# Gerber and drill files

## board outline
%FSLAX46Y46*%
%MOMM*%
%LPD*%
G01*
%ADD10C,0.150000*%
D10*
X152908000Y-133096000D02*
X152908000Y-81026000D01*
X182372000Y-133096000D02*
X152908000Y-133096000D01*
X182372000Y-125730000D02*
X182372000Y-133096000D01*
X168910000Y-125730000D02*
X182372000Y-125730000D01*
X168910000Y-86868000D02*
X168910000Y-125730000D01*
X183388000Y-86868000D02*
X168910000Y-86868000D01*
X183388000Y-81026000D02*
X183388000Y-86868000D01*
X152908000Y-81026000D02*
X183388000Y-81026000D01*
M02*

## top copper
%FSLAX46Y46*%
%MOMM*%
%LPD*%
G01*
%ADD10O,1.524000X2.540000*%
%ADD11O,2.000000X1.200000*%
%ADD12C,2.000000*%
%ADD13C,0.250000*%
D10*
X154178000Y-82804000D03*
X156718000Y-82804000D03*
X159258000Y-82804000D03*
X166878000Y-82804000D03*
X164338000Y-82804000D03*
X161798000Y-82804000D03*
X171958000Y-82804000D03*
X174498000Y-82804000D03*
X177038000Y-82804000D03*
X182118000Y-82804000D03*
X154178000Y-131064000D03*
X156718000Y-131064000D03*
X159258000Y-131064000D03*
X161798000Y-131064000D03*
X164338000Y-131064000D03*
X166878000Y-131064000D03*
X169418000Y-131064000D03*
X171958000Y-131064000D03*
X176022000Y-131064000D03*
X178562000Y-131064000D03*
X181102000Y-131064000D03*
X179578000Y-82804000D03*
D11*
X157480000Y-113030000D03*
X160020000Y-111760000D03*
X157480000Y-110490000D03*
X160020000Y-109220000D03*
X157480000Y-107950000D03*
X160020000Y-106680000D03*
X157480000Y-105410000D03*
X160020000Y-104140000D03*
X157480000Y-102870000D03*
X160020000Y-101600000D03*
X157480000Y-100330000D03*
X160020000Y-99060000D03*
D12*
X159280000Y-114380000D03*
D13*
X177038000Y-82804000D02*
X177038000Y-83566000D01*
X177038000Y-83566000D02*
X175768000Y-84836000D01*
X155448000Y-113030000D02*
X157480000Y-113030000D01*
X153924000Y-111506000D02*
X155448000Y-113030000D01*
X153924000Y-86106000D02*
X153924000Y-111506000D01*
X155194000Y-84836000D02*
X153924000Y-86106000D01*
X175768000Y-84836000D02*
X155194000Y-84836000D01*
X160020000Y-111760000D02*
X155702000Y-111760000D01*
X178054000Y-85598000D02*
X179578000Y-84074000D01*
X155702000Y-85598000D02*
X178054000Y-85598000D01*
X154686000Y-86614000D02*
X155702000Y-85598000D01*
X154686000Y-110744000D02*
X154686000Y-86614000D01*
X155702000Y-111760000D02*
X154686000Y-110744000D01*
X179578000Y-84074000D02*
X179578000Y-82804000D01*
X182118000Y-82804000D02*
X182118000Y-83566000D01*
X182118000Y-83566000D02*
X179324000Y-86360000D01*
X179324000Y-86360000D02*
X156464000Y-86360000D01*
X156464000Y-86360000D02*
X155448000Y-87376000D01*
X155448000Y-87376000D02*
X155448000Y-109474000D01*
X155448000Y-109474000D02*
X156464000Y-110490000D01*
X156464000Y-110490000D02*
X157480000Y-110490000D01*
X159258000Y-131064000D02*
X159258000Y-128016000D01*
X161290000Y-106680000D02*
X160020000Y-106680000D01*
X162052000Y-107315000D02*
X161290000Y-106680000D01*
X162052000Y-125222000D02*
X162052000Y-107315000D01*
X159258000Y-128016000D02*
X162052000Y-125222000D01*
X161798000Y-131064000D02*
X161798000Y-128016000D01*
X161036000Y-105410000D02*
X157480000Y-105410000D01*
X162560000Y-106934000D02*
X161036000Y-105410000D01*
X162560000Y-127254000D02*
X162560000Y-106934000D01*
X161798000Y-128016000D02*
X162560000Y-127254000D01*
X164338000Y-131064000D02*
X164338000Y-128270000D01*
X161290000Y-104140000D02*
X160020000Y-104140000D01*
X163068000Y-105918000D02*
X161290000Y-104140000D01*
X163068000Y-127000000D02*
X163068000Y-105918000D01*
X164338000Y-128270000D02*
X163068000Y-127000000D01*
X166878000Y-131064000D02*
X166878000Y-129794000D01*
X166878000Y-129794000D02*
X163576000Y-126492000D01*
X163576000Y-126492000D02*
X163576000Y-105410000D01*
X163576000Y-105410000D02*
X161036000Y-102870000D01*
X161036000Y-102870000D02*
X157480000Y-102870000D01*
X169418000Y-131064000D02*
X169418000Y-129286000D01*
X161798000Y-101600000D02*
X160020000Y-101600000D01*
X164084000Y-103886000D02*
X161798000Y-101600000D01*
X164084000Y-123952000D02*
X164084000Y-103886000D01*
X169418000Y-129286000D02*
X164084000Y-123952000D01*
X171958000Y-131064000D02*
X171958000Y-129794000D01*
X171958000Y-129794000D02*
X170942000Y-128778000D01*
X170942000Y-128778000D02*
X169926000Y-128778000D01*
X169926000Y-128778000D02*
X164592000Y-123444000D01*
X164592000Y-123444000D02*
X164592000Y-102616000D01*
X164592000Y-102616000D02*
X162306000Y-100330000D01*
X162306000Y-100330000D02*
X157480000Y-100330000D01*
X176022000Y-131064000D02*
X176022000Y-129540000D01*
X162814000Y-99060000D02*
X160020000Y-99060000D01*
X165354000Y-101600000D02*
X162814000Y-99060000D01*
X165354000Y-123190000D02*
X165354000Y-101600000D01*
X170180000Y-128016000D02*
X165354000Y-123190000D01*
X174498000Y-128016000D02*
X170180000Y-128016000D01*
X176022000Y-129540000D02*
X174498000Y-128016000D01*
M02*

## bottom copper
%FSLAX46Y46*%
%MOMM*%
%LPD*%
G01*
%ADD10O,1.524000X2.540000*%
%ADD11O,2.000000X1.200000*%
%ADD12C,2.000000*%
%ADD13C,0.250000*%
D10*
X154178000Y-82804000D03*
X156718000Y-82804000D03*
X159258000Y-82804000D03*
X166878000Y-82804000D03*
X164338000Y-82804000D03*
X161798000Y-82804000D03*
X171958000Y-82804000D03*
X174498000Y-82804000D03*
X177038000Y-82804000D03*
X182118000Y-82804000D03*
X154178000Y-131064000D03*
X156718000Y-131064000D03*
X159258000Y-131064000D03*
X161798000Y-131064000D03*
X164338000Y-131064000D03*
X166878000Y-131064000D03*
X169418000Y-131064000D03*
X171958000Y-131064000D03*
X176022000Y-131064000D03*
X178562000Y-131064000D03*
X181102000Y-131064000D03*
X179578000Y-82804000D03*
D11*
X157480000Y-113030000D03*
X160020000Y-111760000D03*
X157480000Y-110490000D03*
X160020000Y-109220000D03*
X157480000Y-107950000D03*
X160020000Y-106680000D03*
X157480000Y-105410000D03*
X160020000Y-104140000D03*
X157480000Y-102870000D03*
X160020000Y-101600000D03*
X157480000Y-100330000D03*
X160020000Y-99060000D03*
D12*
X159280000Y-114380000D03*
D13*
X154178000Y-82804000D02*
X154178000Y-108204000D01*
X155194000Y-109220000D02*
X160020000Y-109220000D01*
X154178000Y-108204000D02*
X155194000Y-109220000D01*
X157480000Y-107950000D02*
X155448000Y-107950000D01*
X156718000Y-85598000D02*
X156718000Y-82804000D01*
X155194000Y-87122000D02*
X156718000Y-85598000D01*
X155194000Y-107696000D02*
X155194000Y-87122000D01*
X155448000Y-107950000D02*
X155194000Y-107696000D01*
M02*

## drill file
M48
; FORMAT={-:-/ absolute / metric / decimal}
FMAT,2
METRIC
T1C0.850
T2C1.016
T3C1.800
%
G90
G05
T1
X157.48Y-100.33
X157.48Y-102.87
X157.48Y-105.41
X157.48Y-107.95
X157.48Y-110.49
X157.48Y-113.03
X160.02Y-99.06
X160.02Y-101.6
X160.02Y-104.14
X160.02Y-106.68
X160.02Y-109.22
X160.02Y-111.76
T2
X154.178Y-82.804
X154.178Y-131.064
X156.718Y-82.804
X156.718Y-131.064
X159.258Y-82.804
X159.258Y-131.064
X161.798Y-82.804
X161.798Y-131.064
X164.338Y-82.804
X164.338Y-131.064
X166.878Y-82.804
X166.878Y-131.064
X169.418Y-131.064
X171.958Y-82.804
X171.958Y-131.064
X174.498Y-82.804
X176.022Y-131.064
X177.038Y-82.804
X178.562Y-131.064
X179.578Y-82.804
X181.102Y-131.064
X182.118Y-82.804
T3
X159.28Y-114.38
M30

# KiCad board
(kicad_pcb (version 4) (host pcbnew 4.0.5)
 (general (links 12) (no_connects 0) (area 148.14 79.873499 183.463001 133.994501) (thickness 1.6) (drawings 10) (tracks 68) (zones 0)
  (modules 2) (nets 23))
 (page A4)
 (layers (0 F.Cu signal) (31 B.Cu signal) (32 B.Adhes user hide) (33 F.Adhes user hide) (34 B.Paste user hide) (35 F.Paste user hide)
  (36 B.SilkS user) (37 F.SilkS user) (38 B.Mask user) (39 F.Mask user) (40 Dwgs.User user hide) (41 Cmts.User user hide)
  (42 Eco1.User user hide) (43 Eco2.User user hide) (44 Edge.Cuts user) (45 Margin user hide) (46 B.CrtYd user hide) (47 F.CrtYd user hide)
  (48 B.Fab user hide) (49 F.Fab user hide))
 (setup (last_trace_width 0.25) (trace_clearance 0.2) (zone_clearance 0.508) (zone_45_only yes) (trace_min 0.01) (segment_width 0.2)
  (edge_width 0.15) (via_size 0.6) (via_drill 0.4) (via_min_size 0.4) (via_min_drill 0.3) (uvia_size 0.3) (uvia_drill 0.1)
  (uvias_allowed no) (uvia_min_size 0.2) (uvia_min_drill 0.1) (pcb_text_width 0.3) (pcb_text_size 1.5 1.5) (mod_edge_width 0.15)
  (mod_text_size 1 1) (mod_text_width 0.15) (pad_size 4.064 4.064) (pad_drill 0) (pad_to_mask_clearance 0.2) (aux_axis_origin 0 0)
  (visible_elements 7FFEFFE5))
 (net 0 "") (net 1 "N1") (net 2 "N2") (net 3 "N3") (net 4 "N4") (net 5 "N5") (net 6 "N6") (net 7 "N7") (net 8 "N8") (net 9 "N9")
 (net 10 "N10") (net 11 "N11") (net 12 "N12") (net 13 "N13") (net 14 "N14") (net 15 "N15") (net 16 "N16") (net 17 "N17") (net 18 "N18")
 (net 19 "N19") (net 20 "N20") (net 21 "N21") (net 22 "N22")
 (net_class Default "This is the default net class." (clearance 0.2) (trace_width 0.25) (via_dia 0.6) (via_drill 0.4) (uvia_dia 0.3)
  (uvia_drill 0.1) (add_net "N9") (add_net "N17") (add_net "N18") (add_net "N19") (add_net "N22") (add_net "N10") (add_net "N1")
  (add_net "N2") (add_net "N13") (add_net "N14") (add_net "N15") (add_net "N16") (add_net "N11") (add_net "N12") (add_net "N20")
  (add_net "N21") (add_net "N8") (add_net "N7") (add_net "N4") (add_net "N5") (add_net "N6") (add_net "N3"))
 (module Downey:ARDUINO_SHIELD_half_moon (layer F.Cu) (at 148.59 104.14 270)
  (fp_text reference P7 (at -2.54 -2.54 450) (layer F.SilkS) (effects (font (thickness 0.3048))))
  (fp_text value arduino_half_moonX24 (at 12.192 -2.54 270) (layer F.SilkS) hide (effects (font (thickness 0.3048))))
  (pad 11 thru_hole oval (at -21.336 -5.588 270) (size 2.54 1.524) (drill 1.016) (layers *.Cu *.Mask F.SilkS) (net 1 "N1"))
  (pad 10 thru_hole oval (at -21.336 -8.128 270) (size 2.54 1.524) (drill 1.016) (layers *.Cu *.Mask F.SilkS) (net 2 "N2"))
  (pad 9 thru_hole oval (at -21.336 -10.668 270) (size 2.54 1.524) (drill 1.016) (layers *.Cu *.Mask F.SilkS) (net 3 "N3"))
  (pad 6 thru_hole oval (at -21.336 -18.288 270) (size 2.54 1.524) (drill 1.016) (layers *.Cu *.Mask F.SilkS) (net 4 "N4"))
  (pad 7 thru_hole oval (at -21.336 -15.748 270) (size 2.54 1.524) (drill 1.016) (layers *.Cu *.Mask F.SilkS) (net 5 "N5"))
  (pad 8 thru_hole oval (at -21.336 -13.208 270) (size 2.54 1.524) (drill 1.016) (layers *.Cu *.Mask F.SilkS) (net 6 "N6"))
  (pad 5 thru_hole oval (at -21.336 -23.368 270) (size 2.54 1.524) (drill 1.016) (layers *.Cu *.Mask F.SilkS) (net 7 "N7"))
  (pad 4 thru_hole oval (at -21.336 -25.908 270) (size 2.54 1.524) (drill 1.016) (layers *.Cu *.Mask F.SilkS) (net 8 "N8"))
  (pad 3 thru_hole oval (at -21.336 -28.448 270) (size 2.54 1.524) (drill 1.016) (layers *.Cu *.Mask F.SilkS) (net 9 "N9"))
  (pad 1 thru_hole oval (at -21.336 -33.528 270) (size 2.54 1.524) (drill 1.016) (layers *.Cu *.Mask F.SilkS) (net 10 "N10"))
  (pad 12 thru_hole oval (at 26.924 -5.588 270) (size 2.54 1.524) (drill 1.016) (layers *.Cu *.Mask F.SilkS) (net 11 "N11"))
  (pad 13 thru_hole oval (at 26.924 -8.128 270) (size 2.54 1.524) (drill 1.016) (layers *.Cu *.Mask F.SilkS) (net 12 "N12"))
  (pad 14 thru_hole oval (at 26.924 -10.668 270) (size 2.54 1.524) (drill 1.016) (layers *.Cu *.Mask F.SilkS) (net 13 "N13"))
  (pad 15 thru_hole oval (at 26.924 -13.208 270) (size 2.54 1.524) (drill 1.016) (layers *.Cu *.Mask F.SilkS) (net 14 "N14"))
  (pad 16 thru_hole oval (at 26.924 -15.748 270) (size 2.54 1.524) (drill 1.016) (layers *.Cu *.Mask F.SilkS) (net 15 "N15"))
  (pad 17 thru_hole oval (at 26.924 -18.288 270) (size 2.54 1.524) (drill 1.016) (layers *.Cu *.Mask F.SilkS) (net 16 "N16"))
  (pad 18 thru_hole oval (at 26.924 -20.828 270) (size 2.54 1.524) (drill 1.016) (layers *.Cu *.Mask F.SilkS) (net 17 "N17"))
  (pad 19 thru_hole oval (at 26.924 -23.368 270) (size 2.54 1.524) (drill 1.016) (layers *.Cu *.Mask F.SilkS) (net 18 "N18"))
  (pad 20 thru_hole oval (at 26.924 -27.432 270) (size 2.54 1.524) (drill 1.016) (layers *.Cu *.Mask F.SilkS) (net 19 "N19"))
  (pad 21 thru_hole oval (at 26.924 -29.972 270) (size 2.54 1.524) (drill 1.016) (layers *.Cu *.Mask F.SilkS) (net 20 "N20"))
  (pad 22 thru_hole oval (at 26.924 -32.512 270) (size 2.54 1.524) (drill 1.016) (layers *.Cu *.Mask F.SilkS) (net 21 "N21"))
  (pad 2 thru_hole oval (at -21.336 -30.988 270) (size 2.54 1.524) (drill 1.016) (layers *.Cu *.Mask F.SilkS) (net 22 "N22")))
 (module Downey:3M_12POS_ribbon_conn (layer F.Cu) (at 158.75 106.68 90)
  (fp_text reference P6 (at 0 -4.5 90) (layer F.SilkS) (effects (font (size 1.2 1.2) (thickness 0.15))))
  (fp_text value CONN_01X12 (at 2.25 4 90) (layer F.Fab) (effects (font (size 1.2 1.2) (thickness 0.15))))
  (pad 1 thru_hole oval (at -6.35 -1.27 90) (size 1.2 2) (drill 0.85) (layers *.Cu *.Mask) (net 9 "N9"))
  (pad 2 thru_hole oval (at -5.08 1.27 90) (size 1.2 2) (drill 0.85) (layers *.Cu *.Mask) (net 22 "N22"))
  (pad 3 thru_hole oval (at -3.81 -1.27 90) (size 1.2 2) (drill 0.85) (layers *.Cu *.Mask) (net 10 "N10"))
  (pad 4 thru_hole oval (at -2.54 1.27 90) (size 1.2 2) (drill 0.85) (layers *.Cu *.Mask) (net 1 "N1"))
  (pad 5 thru_hole oval (at -1.27 -1.27 90) (size 1.2 2) (drill 0.85) (layers *.Cu *.Mask) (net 2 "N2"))
  (pad 6 thru_hole oval (at 0 1.27 90) (size 1.2 2) (drill 0.85) (layers *.Cu *.Mask) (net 13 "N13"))
  (pad 7 thru_hole oval (at 1.27 -1.27 90) (size 1.2 2) (drill 0.85) (layers *.Cu *.Mask) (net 14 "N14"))
  (pad 8 thru_hole oval (at 2.54 1.27 90) (size 1.2 2) (drill 0.85) (layers *.Cu *.Mask) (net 15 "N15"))
  (pad 9 thru_hole oval (at 3.81 -1.27 90) (size 1.2 2) (drill 0.85) (layers *.Cu *.Mask) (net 16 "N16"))
  (pad 10 thru_hole oval (at 5.08 1.27 90) (size 1.2 2) (drill 0.85) (layers *.Cu *.Mask) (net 17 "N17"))
  (pad 11 thru_hole oval (at 6.35 -1.27 90) (size 1.2 2) (drill 0.85) (layers *.Cu *.Mask) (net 18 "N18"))
  (pad 12 thru_hole oval (at 7.62 1.27 90) (size 1.2 2) (drill 0.85) (layers *.Cu *.Mask) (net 19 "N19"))
  (pad "" np_thru_hole circle (at -7.7 0.53 90) (size 2 2) (drill 1.8) (layers *.Cu *.Mask)))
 (gr_line (start 152.908 133.096) (end 152.908 81.026) (angle 90) (layer Edge.Cuts) (width 0.15))
 (gr_line (start 182.372 133.096) (end 152.908 133.096) (angle 90) (layer Edge.Cuts) (width 0.15))
 (gr_line (start 182.372 125.73) (end 182.372 133.096) (angle 90) (layer Edge.Cuts) (width 0.15))
 (gr_line (start 168.91 125.73) (end 182.372 125.73) (angle 90) (layer Edge.Cuts) (width 0.15))
 (gr_line (start 168.91 86.868) (end 168.91 125.73) (angle 90) (layer Edge.Cuts) (width 0.15))
 (gr_line (start 183.388 86.868) (end 168.91 86.868) (angle 90) (layer Edge.Cuts) (width 0.15))
 (gr_line (start 183.388 81.026) (end 183.388 86.868) (angle 90) (layer Edge.Cuts) (width 0.15))
 (gr_line (start 152.908 81.026) (end 183.388 81.026) (angle 90) (layer Edge.Cuts) (width 0.15))
 (segment (start 177.038 82.804) (end 177.038 83.566) (width 0.25) (layer F.Cu) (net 9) (status C00000))
 (segment (start 177.038 83.566) (end 175.768 84.836) (width 0.25) (layer F.Cu) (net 9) (status 400000))
 (segment (start 155.448 113.03) (end 157.48 113.03) (width 0.25) (layer F.Cu) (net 9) (status 800000))
 (segment (start 153.924 111.506) (end 155.448 113.03) (width 0.25) (layer F.Cu) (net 9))
 (segment (start 153.924 86.106) (end 153.924 111.506) (width 0.25) (layer F.Cu) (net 9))
 (segment (start 155.194 84.836) (end 153.924 86.106) (width 0.25) (layer F.Cu) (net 9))
 (segment (start 175.768 84.836) (end 155.194 84.836) (width 0.25) (layer F.Cu) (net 9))
 (segment (start 160.02 111.76) (end 155.702 111.76) (width 0.25) (layer F.Cu) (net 22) (status 400000))
 (segment (start 178.054 85.598) (end 179.578 84.074) (width 0.25) (layer F.Cu) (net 22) (status 800000))
 (segment (start 155.702 85.598) (end 178.054 85.598) (width 0.25) (layer F.Cu) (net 22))
 (segment (start 154.686 86.614) (end 155.702 85.598) (width 0.25) (layer F.Cu) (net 22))
 (segment (start 154.686 110.744) (end 154.686 86.614) (width 0.25) (layer F.Cu) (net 22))
 (segment (start 155.702 111.76) (end 154.686 110.744) (width 0.25) (layer F.Cu) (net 22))
 (segment (start 179.578 84.074) (end 179.578 82.804) (width 0.25) (layer F.Cu) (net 22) (status C00000))
 (segment (start 182.118 82.804) (end 182.118 83.566) (width 0.25) (layer F.Cu) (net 10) (status C00000))
 (segment (start 182.118 83.566) (end 179.324 86.36) (width 0.25) (layer F.Cu) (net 10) (status 400000))
 (segment (start 179.324 86.36) (end 156.464 86.36) (width 0.25) (layer F.Cu) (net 10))
 (segment (start 156.464 86.36) (end 155.448 87.376) (width 0.25) (layer F.Cu) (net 10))
 (segment (start 155.448 87.376) (end 155.448 109.474) (width 0.25) (layer F.Cu) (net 10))
 (segment (start 155.448 109.474) (end 156.464 110.49) (width 0.25) (layer F.Cu) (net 10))
 (segment (start 156.464 110.49) (end 157.48 110.49) (width 0.25) (layer F.Cu) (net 10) (status 800000))
 (segment (start 154.178 82.804) (end 154.178 108.204) (width 0.25) (layer B.Cu) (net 1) (status 400000))
 (segment (start 155.194 109.22) (end 160.02 109.22) (width 0.25) (layer B.Cu) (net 1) (status 800000))
 (segment (start 154.178 108.204) (end 155.194 109.22) (width 0.25) (layer B.Cu) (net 1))
 (segment (start 157.48 107.95) (end 155.448 107.95) (width 0.25) (layer B.Cu) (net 2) (status 400000))
 (segment (start 156.718 85.598) (end 156.718 82.804) (width 0.25) (layer B.Cu) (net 2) (status 800000))
 (segment (start 155.194 87.122) (end 156.718 85.598) (width 0.25) (layer B.Cu) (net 2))
 (segment (start 155.194 107.696) (end 155.194 87.122) (width 0.25) (layer B.Cu) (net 2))
 (segment (start 155.448 107.95) (end 155.194 107.696) (width 0.25) (layer B.Cu) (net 2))
 (segment (start 159.258 131.064) (end 159.258 128.016) (width 0.25) (layer F.Cu) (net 13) (status 10))
 (segment (start 161.29 106.68) (end 160.02 106.68) (width 0.25) (layer F.Cu) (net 13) (status 20))
 (segment (start 162.052 107.315) (end 161.29 106.68) (width 0.25) (layer F.Cu) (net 13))
 (segment (start 162.052 125.222) (end 162.052 107.315) (width 0.25) (layer F.Cu) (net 13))
 (segment (start 159.258 128.016) (end 162.052 125.222) (width 0.25) (layer F.Cu) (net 13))
 (segment (start 161.798 131.064) (end 161.798 128.016) (width 0.25) (layer F.Cu) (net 14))
 (segment (start 161.036 105.41) (end 157.48 105.41) (width 0.25) (layer F.Cu) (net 14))
 (segment (start 162.56 106.934) (end 161.036 105.41) (width 0.25) (layer F.Cu) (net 14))
 (segment (start 162.56 127.254) (end 162.56 106.934) (width 0.25) (layer F.Cu) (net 14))
 (segment (start 161.798 128.016) (end 162.56 127.254) (width 0.25) (layer F.Cu) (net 14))
 (segment (start 164.338 131.064) (end 164.338 128.27) (width 0.25) (layer F.Cu) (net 15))
 (segment (start 161.29 104.14) (end 160.02 104.14) (width 0.25) (layer F.Cu) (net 15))
 (segment (start 163.068 105.918) (end 161.29 104.14) (width 0.25) (layer F.Cu) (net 15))
 (segment (start 163.068 127) (end 163.068 105.918) (width 0.25) (layer F.Cu) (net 15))
 (segment (start 164.338 128.27) (end 163.068 127) (width 0.25) (layer F.Cu) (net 15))
 (segment (start 166.878 131.064) (end 166.878 129.794) (width 0.25) (layer F.Cu) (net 16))
 (segment (start 166.878 129.794) (end 163.576 126.492) (width 0.25) (layer F.Cu) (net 16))
 (segment (start 163.576 126.492) (end 163.576 105.41) (width 0.25) (layer F.Cu) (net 16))
 (segment (start 163.576 105.41) (end 161.036 102.87) (width 0.25) (layer F.Cu) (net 16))
 (segment (start 161.036 102.87) (end 157.48 102.87) (width 0.25) (layer F.Cu) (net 16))
 (segment (start 169.418 131.064) (end 169.418 129.286) (width 0.25) (layer F.Cu) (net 17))
 (segment (start 161.798 101.6) (end 160.02 101.6) (width 0.25) (layer F.Cu) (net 17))
 (segment (start 164.084 103.886) (end 161.798 101.6) (width 0.25) (layer F.Cu) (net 17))
 (segment (start 164.084 123.952) (end 164.084 103.886) (width 0.25) (layer F.Cu) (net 17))
 (segment (start 169.418 129.286) (end 164.084 123.952) (width 0.25) (layer F.Cu) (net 17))
 (segment (start 171.958 131.064) (end 171.958 129.794) (width 0.25) (layer F.Cu) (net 18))
 (segment (start 171.958 129.794) (end 170.942 128.778) (width 0.25) (layer F.Cu) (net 18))
 (segment (start 170.942 128.778) (end 169.926 128.778) (width 0.25) (layer F.Cu) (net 18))
 (segment (start 169.926 128.778) (end 164.592 123.444) (width 0.25) (layer F.Cu) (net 18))
 (segment (start 164.592 123.444) (end 164.592 102.616) (width 0.25) (layer F.Cu) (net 18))
 (segment (start 164.592 102.616) (end 162.306 100.33) (width 0.25) (layer F.Cu) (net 18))
 (segment (start 162.306 100.33) (end 157.48 100.33) (width 0.25) (layer F.Cu) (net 18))
 (segment (start 176.022 131.064) (end 176.022 129.54) (width 0.25) (layer F.Cu) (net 19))
 (segment (start 162.814 99.06) (end 160.02 99.06) (width 0.25) (layer F.Cu) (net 19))
 (segment (start 165.354 101.6) (end 162.814 99.06) (width 0.25) (layer F.Cu) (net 19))
 (segment (start 165.354 123.19) (end 165.354 101.6) (width 0.25) (layer F.Cu) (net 19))
 (segment (start 170.18 128.016) (end 165.354 123.19) (width 0.25) (layer F.Cu) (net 19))
 (segment (start 174.498 128.016) (end 170.18 128.016) (width 0.25) (layer F.Cu) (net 19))
 (segment (start 176.022 129.54) (end 174.498 128.016) (width 0.25) (layer F.Cu) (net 19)))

